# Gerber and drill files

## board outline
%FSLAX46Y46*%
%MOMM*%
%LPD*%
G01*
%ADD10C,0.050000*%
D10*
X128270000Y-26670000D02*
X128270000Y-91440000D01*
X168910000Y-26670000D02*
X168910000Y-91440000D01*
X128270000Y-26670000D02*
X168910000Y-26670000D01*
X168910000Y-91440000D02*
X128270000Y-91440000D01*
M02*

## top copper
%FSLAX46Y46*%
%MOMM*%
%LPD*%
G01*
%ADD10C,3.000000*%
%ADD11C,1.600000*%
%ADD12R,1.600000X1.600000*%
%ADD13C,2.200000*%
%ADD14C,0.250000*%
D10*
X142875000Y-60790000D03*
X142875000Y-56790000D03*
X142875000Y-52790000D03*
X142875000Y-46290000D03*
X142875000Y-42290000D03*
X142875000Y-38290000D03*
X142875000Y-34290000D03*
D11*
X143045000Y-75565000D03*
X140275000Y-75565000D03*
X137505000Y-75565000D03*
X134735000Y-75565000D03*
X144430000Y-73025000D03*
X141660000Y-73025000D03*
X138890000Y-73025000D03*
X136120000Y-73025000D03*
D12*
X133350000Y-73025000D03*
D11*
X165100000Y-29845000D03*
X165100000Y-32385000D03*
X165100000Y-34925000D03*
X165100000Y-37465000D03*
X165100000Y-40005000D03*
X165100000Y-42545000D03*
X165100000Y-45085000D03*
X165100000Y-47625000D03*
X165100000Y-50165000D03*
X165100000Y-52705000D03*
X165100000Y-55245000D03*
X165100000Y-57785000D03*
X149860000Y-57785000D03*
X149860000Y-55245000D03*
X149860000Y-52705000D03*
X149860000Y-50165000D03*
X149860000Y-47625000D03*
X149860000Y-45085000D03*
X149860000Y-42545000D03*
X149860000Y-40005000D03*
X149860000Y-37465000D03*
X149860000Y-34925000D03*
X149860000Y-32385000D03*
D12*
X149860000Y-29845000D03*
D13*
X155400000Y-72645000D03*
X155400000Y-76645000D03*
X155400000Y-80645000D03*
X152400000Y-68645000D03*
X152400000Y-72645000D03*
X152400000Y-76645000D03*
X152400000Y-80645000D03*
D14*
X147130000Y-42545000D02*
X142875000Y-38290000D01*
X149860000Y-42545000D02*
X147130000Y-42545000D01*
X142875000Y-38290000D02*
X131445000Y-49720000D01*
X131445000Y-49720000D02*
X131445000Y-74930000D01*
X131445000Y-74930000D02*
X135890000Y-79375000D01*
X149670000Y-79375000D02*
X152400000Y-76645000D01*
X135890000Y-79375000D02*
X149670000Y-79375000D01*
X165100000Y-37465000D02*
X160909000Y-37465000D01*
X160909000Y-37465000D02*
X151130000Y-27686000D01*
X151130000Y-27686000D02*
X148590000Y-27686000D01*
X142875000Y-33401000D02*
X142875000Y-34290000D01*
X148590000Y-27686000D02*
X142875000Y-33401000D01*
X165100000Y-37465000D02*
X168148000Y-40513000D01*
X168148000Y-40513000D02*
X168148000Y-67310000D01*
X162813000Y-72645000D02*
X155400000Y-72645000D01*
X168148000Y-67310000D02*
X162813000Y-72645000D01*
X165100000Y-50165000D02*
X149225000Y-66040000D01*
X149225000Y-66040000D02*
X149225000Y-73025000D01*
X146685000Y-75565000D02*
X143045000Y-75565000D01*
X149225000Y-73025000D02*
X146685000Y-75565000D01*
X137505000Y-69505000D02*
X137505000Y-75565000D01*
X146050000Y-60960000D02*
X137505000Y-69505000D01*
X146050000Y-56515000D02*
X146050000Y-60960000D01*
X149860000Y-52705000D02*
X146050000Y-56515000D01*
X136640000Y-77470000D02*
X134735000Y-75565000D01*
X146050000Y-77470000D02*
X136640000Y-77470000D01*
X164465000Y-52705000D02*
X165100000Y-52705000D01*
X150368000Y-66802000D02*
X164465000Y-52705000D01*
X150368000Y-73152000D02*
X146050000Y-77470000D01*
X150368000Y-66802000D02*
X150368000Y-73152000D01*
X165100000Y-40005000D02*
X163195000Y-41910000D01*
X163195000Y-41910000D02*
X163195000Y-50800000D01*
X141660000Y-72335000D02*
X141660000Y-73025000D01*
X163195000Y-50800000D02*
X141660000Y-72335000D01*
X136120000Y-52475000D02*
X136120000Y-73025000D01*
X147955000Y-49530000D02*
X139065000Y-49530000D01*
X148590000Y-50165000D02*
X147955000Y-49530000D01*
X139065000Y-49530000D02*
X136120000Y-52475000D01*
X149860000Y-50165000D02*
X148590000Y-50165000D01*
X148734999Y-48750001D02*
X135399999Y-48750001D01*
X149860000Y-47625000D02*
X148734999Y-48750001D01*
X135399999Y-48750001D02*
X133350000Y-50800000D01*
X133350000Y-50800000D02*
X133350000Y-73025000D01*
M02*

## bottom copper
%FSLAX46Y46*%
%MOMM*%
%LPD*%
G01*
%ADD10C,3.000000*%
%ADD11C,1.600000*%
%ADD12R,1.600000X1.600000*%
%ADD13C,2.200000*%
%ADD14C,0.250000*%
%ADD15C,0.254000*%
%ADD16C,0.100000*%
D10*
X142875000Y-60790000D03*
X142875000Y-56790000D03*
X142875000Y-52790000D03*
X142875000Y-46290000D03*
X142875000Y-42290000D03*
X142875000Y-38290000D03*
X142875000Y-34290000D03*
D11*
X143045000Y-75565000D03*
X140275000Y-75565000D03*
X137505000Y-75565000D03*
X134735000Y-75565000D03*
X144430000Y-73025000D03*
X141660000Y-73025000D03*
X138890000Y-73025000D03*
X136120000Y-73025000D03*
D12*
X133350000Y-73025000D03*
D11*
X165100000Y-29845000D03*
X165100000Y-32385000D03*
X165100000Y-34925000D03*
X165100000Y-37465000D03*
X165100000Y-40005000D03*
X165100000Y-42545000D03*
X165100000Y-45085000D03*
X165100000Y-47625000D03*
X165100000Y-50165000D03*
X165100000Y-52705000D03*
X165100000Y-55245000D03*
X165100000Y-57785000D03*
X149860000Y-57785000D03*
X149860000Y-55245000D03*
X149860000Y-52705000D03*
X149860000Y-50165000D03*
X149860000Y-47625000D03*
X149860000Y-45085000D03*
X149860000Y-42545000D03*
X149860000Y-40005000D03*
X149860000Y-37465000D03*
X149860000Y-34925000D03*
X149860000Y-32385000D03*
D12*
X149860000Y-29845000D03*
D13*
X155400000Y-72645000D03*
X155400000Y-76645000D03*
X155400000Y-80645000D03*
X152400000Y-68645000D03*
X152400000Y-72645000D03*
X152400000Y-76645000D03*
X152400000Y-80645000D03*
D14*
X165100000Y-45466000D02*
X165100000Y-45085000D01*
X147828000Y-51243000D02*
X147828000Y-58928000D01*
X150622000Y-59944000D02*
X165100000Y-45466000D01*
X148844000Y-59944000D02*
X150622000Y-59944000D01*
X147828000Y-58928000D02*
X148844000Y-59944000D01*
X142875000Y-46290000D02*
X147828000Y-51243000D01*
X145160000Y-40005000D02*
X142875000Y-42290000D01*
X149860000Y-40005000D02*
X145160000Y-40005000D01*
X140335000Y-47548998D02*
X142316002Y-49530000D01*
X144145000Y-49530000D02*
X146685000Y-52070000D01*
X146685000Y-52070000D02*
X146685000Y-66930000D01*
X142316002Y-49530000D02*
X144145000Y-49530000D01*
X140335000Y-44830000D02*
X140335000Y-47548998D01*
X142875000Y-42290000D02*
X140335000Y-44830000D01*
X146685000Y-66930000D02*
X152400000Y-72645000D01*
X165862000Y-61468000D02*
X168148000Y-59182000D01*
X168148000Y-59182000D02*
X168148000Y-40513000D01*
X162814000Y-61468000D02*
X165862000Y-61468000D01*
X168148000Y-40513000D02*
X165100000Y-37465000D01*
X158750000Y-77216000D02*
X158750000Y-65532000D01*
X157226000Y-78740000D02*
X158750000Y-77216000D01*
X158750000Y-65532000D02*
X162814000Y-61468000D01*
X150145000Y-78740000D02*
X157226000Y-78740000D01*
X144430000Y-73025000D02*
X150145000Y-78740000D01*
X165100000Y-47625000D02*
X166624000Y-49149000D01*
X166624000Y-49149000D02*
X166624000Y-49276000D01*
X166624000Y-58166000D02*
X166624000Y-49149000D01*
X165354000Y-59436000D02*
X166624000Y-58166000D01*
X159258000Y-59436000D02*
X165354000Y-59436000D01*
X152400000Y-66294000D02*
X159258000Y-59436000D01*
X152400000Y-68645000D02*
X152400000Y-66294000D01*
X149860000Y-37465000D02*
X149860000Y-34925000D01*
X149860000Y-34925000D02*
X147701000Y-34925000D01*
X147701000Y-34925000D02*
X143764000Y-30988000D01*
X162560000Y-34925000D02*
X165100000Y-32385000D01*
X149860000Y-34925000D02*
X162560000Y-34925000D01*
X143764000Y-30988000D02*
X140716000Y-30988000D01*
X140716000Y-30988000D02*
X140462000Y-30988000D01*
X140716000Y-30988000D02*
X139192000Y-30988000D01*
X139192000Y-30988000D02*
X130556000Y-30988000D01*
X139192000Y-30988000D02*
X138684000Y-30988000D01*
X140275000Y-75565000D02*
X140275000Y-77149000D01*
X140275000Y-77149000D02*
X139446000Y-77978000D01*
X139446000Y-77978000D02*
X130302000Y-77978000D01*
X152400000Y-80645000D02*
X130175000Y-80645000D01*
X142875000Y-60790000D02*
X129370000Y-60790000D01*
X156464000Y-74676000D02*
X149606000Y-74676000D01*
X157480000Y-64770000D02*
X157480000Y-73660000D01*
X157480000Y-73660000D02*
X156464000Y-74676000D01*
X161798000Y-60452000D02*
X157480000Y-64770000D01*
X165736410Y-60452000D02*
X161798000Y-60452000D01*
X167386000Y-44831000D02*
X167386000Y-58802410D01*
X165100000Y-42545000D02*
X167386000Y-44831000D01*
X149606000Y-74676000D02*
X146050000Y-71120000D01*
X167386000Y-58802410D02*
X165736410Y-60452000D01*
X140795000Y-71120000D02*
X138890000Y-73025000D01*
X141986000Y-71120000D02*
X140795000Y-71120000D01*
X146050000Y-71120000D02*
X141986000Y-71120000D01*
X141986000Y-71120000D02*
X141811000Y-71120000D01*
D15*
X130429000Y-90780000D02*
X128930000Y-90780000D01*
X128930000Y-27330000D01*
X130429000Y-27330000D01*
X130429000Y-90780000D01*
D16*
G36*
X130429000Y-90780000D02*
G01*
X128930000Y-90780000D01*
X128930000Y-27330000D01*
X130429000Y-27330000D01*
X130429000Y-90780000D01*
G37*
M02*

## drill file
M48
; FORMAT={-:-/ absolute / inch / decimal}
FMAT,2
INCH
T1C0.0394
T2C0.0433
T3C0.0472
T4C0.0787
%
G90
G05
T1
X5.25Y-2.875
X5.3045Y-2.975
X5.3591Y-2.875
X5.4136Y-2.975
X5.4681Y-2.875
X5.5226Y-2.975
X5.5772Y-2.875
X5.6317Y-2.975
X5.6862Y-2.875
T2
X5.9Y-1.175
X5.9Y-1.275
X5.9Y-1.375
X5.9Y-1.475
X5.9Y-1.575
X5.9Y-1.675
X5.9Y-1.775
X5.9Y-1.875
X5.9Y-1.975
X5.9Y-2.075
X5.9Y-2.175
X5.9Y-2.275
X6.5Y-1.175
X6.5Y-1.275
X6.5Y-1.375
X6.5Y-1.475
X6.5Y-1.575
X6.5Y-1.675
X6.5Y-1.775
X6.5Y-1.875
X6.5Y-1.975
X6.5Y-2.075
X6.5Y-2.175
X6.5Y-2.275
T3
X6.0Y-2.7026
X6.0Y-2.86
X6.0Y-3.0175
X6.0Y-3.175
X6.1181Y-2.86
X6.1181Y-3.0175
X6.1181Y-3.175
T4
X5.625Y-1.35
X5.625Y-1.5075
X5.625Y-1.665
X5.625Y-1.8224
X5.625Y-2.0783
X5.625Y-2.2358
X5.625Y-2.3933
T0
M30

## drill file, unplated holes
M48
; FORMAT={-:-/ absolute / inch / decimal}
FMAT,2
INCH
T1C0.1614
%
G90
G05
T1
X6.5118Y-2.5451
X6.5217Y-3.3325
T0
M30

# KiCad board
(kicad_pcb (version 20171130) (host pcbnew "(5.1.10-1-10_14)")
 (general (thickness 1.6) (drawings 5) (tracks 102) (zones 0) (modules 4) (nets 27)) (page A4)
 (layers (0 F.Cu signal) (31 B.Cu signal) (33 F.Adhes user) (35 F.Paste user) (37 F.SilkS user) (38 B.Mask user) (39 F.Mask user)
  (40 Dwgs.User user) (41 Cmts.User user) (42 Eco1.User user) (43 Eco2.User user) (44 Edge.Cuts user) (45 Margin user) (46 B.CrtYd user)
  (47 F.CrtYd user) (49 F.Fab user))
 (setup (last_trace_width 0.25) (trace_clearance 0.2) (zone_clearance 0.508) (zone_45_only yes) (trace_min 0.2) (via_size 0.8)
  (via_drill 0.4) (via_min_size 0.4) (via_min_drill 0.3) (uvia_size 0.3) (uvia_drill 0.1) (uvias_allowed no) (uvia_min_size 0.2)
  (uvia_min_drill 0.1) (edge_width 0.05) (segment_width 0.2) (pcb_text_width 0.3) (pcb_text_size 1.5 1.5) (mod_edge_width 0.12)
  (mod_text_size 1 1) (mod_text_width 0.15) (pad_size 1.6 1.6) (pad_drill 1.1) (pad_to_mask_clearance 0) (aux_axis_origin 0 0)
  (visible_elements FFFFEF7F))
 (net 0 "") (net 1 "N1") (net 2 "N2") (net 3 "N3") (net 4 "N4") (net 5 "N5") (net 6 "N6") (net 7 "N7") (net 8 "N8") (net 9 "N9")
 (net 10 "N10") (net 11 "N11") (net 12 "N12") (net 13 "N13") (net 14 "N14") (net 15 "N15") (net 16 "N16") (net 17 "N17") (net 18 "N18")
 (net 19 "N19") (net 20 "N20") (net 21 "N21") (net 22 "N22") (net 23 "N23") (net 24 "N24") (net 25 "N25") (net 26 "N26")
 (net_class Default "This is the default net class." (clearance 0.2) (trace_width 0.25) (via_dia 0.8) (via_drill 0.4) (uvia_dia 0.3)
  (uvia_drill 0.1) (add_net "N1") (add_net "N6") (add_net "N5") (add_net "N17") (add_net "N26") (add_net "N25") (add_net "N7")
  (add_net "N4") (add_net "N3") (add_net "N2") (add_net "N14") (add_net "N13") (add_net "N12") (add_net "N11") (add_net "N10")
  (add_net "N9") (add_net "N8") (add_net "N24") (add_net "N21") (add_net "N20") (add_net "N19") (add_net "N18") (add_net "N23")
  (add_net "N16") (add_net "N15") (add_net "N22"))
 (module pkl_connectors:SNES (layer F.Cu) (at 142.875 34.29 270)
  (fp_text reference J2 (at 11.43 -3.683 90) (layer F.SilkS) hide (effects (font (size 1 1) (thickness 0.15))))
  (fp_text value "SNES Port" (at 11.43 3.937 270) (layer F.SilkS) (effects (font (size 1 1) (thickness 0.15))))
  (pad 7 thru_hole circle (at 26.5 0 270) (size 3 3) (drill 2) (layers *.Cu *.Mask) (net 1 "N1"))
  (pad 6 thru_hole circle (at 22.5 0 270) (size 3 3) (drill 2) (layers *.Cu *.Mask) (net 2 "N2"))
  (pad 5 thru_hole circle (at 18.5 0 270) (size 3 3) (drill 2) (layers *.Cu *.Mask) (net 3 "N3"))
  (pad 4 thru_hole circle (at 12 0 270) (size 3 3) (drill 2) (layers *.Cu *.Mask) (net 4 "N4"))
  (pad 3 thru_hole circle (at 8 0 270) (size 3 3) (drill 2) (layers *.Cu *.Mask) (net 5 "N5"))
  (pad 2 thru_hole circle (at 4 0 270) (size 3 3) (drill 2) (layers *.Cu *.Mask) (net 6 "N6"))
  (pad 1 thru_hole circle (at 0 0 270) (size 3 3) (drill 2) (layers *.Cu *.Mask) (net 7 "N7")))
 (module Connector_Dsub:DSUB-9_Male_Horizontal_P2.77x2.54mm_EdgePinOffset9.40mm (layer F.Cu) (at 133.35 73.025)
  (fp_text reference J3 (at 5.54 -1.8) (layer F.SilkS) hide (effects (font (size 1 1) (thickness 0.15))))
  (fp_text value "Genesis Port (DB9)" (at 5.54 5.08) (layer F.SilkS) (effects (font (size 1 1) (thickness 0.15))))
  (pad 9 thru_hole circle (at 9.695 2.54) (size 1.6 1.6) (drill 1) (layers *.Cu *.Mask) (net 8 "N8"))
  (pad 8 thru_hole circle (at 6.925 2.54) (size 1.6 1.6) (drill 1) (layers *.Cu *.Mask) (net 1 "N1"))
  (pad 7 thru_hole circle (at 4.155 2.54) (size 1.6 1.6) (drill 1) (layers *.Cu *.Mask) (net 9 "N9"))
  (pad 6 thru_hole circle (at 1.385 2.54) (size 1.6 1.6) (drill 1) (layers *.Cu *.Mask) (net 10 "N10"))
  (pad 5 thru_hole circle (at 11.08 0) (size 1.6 1.6) (drill 1) (layers *.Cu *.Mask) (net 7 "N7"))
  (pad 4 thru_hole circle (at 8.31 0) (size 1.6 1.6) (drill 1) (layers *.Cu *.Mask) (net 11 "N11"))
  (pad 3 thru_hole circle (at 5.54 0) (size 1.6 1.6) (drill 1) (layers *.Cu *.Mask) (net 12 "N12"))
  (pad 2 thru_hole circle (at 2.77 0) (size 1.6 1.6) (drill 1) (layers *.Cu *.Mask) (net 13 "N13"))
  (pad 1 thru_hole rect (at 0 0) (size 1.6 1.6) (drill 1) (layers *.Cu *.Mask) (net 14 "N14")))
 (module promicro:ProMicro (layer F.Cu) (at 157.48 43.815 270)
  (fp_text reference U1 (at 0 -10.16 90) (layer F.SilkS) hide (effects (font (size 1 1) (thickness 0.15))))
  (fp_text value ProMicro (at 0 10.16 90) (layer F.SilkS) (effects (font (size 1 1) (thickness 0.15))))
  (pad 24 thru_hole circle (at -13.97 -7.62 270) (size 1.6 1.6) (drill 1.1) (layers *.Cu *.Mask F.SilkS) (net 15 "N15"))
  (pad 23 thru_hole circle (at -11.43 -7.62 270) (size 1.6 1.6) (drill 1.1) (layers *.Cu *.Mask F.SilkS) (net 1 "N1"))
  (pad 22 thru_hole circle (at -8.89 -7.62 270) (size 1.6 1.6) (drill 1.1) (layers *.Cu *.Mask F.SilkS) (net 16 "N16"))
  (pad 21 thru_hole circle (at -6.35 -7.62 270) (size 1.6 1.6) (drill 1.1) (layers *.Cu *.Mask F.SilkS) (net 7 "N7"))
  (pad 20 thru_hole circle (at -3.81 -7.62 270) (size 1.6 1.6) (drill 1.1) (layers *.Cu *.Mask F.SilkS) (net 11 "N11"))
  (pad 19 thru_hole circle (at -1.27 -7.62 270) (size 1.6 1.6) (drill 1.1) (layers *.Cu *.Mask F.SilkS) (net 12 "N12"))
  (pad 18 thru_hole circle (at 1.27 -7.62 270) (size 1.6 1.6) (drill 1.1) (layers *.Cu *.Mask F.SilkS) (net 4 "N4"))
  (pad 17 thru_hole circle (at 3.81 -7.62 270) (size 1.6 1.6) (drill 1.1) (layers *.Cu *.Mask F.SilkS) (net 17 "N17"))
  (pad 16 thru_hole circle (at 6.35 -7.62 270) (size 1.6 1.6) (drill 1.1) (layers *.Cu *.Mask F.SilkS) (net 8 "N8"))
  (pad 15 thru_hole circle (at 8.89 -7.62 270) (size 1.6 1.6) (drill 1.1) (layers *.Cu *.Mask F.SilkS) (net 10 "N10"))
  (pad 14 thru_hole circle (at 11.43 -7.62 270) (size 1.6 1.6) (drill 1.1) (layers *.Cu *.Mask F.SilkS) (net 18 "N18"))
  (pad 13 thru_hole circle (at 13.97 -7.62 270) (size 1.6 1.6) (drill 1.1) (layers *.Cu *.Mask F.SilkS) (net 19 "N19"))
  (pad 12 thru_hole circle (at 13.97 7.62 270) (size 1.6 1.6) (drill 1.1) (layers *.Cu *.Mask F.SilkS) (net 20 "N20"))
  (pad 11 thru_hole circle (at 11.43 7.62 270) (size 1.6 1.6) (drill 1.1) (layers *.Cu *.Mask F.SilkS) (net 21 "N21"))
  (pad 10 thru_hole circle (at 8.89 7.62 270) (size 1.6 1.6) (drill 1.1) (layers *.Cu *.Mask F.SilkS) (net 9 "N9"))
  (pad 9 thru_hole circle (at 6.35 7.62 270) (size 1.6 1.6) (drill 1.1) (layers *.Cu *.Mask F.SilkS) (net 13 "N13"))
  (pad 8 thru_hole circle (at 3.81 7.62 270) (size 1.6 1.6) (drill 1.1) (layers *.Cu *.Mask F.SilkS) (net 14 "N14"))
  (pad 7 thru_hole circle (at 1.27 7.62 270) (size 1.6 1.6) (drill 1.1) (layers *.Cu *.Mask F.SilkS) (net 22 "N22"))
  (pad 6 thru_hole circle (at -1.27 7.62 270) (size 1.6 1.6) (drill 1.1) (layers *.Cu *.Mask F.SilkS) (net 6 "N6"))
  (pad 5 thru_hole circle (at -3.81 7.62 270) (size 1.6 1.6) (drill 1.1) (layers *.Cu *.Mask F.SilkS) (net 5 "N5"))
  (pad 4 thru_hole circle (at -6.35 7.62 270) (size 1.6 1.6) (drill 1.1) (layers *.Cu *.Mask F.SilkS) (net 1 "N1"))
  (pad 3 thru_hole circle (at -8.89 7.62 270) (size 1.6 1.6) (drill 1.1) (layers *.Cu *.Mask F.SilkS) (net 1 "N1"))
  (pad 2 thru_hole circle (at -11.43 7.62 270) (size 1.6 1.6) (drill 1.1) (layers *.Cu *.Mask F.SilkS) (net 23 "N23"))
  (pad 1 thru_hole rect (at -13.97 7.62 270) (size 1.6 1.6) (drill 1.1) (layers *.Cu *.Mask F.SilkS) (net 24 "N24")))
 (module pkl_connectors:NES (layer F.Cu) (at 152.4 80.645 90)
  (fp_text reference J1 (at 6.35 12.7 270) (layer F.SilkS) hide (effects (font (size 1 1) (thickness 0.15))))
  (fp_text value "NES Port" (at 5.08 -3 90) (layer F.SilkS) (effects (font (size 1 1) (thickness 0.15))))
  (pad "" np_thru_hole circle (at -4 13.25 90) (size 4.1 4.1) (drill 4.1) (layers *.Cu *.Mask))
  (pad "" np_thru_hole circle (at 16 13 90) (size 4.1 4.1) (drill 4.1) (layers *.Cu *.Mask))
  (pad 7 thru_hole circle (at 8 3 90) (size 2.2 2.2) (drill 1.2) (layers *.Cu *.Mask) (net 7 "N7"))
  (pad 6 thru_hole circle (at 4 3 90) (size 2.2 2.2) (drill 1.2) (layers *.Cu *.Mask) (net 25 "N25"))
  (pad 5 thru_hole circle (at 0 3 90) (size 2.2 2.2) (drill 1.2) (layers *.Cu *.Mask) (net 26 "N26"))
  (pad 4 thru_hole circle (at 12 0 90) (size 2.2 2.2) (drill 1.2) (layers *.Cu *.Mask) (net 17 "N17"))
  (pad 3 thru_hole circle (at 8 0 90) (size 2.2 2.2) (drill 1.2) (layers *.Cu *.Mask) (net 5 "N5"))
  (pad 2 thru_hole circle (at 4 0 90) (size 2.2 2.2) (drill 1.2) (layers *.Cu *.Mask) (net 6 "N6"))
  (pad 1 thru_hole circle (at 0 0 90) (size 2.2 2.2) (drill 1.2) (layers *.Cu *.Mask) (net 1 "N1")))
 (gr_line (start 128.27 26.67) (end 128.27 91.44) (layer Edge.Cuts) (width 0.05))
 (gr_line (start 168.91 26.67) (end 168.91 91.44) (layer Edge.Cuts) (width 0.05))
 (gr_line (start 128.27 26.67) (end 168.91 26.67) (layer Edge.Cuts) (width 0.05))
 (gr_line (start 168.91 91.44) (end 128.27 91.44) (layer Edge.Cuts) (width 0.05))
 (segment (start 165.1 45.466) (end 165.1 45.085) (width 0.25) (layer B.Cu) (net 4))
 (segment (start 147.828 51.243) (end 147.828 58.928) (width 0.25) (layer B.Cu) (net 4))
 (segment (start 150.622 59.944) (end 165.1 45.466) (width 0.25) (layer B.Cu) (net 4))
 (segment (start 148.844 59.944) (end 150.622 59.944) (width 0.25) (layer B.Cu) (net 4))
 (segment (start 147.828 58.928) (end 148.844 59.944) (width 0.25) (layer B.Cu) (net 4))
 (segment (start 142.875 46.29) (end 147.828 51.243) (width 0.25) (layer B.Cu) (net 4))
 (segment (start 145.16 40.005) (end 142.875 42.29) (width 0.25) (layer B.Cu) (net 5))
 (segment (start 149.86 40.005) (end 145.16 40.005) (width 0.25) (layer B.Cu) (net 5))
 (segment (start 140.335 47.548998) (end 142.316002 49.53) (width 0.25) (layer B.Cu) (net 5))
 (segment (start 144.145 49.53) (end 146.685 52.07) (width 0.25) (layer B.Cu) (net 5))
 (segment (start 146.685 52.07) (end 146.685 66.93) (width 0.25) (layer B.Cu) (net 5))
 (segment (start 142.316002 49.53) (end 144.145 49.53) (width 0.25) (layer B.Cu) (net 5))
 (segment (start 140.335 44.83) (end 140.335 47.548998) (width 0.25) (layer B.Cu) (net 5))
 (segment (start 142.875 42.29) (end 140.335 44.83) (width 0.25) (layer B.Cu) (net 5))
 (segment (start 146.685 66.93) (end 152.4 72.645) (width 0.25) (layer B.Cu) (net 5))
 (segment (start 147.13 42.545) (end 142.875 38.29) (width 0.25) (layer F.Cu) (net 6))
 (segment (start 149.86 42.545) (end 147.13 42.545) (width 0.25) (layer F.Cu) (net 6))
 (segment (start 142.875 38.29) (end 131.445 49.72) (width 0.25) (layer F.Cu) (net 6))
 (segment (start 131.445 49.72) (end 131.445 74.93) (width 0.25) (layer F.Cu) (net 6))
 (segment (start 131.445 74.93) (end 135.89 79.375) (width 0.25) (layer F.Cu) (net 6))
 (segment (start 149.67 79.375) (end 152.4 76.645) (width 0.25) (layer F.Cu) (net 6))
 (segment (start 135.89 79.375) (end 149.67 79.375) (width 0.25) (layer F.Cu) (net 6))
 (segment (start 165.1 37.465) (end 160.909 37.465) (width 0.25) (layer F.Cu) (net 7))
 (segment (start 160.909 37.465) (end 151.13 27.686) (width 0.25) (layer F.Cu) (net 7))
 (segment (start 151.13 27.686) (end 148.59 27.686) (width 0.25) (layer F.Cu) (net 7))
 (segment (start 142.875 33.401) (end 142.875 34.29) (width 0.25) (layer F.Cu) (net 7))
 (segment (start 148.59 27.686) (end 142.875 33.401) (width 0.25) (layer F.Cu) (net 7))
 (segment (start 165.1 37.465) (end 168.148 40.513) (width 0.25) (layer F.Cu) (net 7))
 (segment (start 168.148 40.513) (end 168.148 67.31) (width 0.25) (layer F.Cu) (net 7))
 (segment (start 162.813 72.645) (end 155.4 72.645) (width 0.25) (layer F.Cu) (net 7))
 (segment (start 168.148 67.31) (end 162.813 72.645) (width 0.25) (layer F.Cu) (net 7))
 (segment (start 165.862 61.468) (end 168.148 59.182) (width 0.25) (layer B.Cu) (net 7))
 (segment (start 168.148 59.182) (end 168.148 40.513) (width 0.25) (layer B.Cu) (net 7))
 (segment (start 162.814 61.468) (end 165.862 61.468) (width 0.25) (layer B.Cu) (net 7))
 (segment (start 168.148 40.513) (end 165.1 37.465) (width 0.25) (layer B.Cu) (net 7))
 (segment (start 158.75 77.216) (end 158.75 65.532) (width 0.25) (layer B.Cu) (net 7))
 (segment (start 157.226 78.74) (end 158.75 77.216) (width 0.25) (layer B.Cu) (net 7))
 (segment (start 158.75 65.532) (end 162.814 61.468) (width 0.25) (layer B.Cu) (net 7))
 (segment (start 150.145 78.74) (end 157.226 78.74) (width 0.25) (layer B.Cu) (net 7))
 (segment (start 144.43 73.025) (end 150.145 78.74) (width 0.25) (layer B.Cu) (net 7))
 (segment (start 165.1 47.625) (end 166.624 49.149) (width 0.25) (layer B.Cu) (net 17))
 (segment (start 166.624 49.149) (end 166.624 49.276) (width 0.25) (layer B.Cu) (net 17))
 (segment (start 166.624 58.166) (end 166.624 49.149) (width 0.25) (layer B.Cu) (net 17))
 (segment (start 165.354 59.436) (end 166.624 58.166) (width 0.25) (layer B.Cu) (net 17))
 (segment (start 159.258 59.436) (end 165.354 59.436) (width 0.25) (layer B.Cu) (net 17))
 (segment (start 152.4 66.294) (end 159.258 59.436) (width 0.25) (layer B.Cu) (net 17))
 (segment (start 152.4 68.645) (end 152.4 66.294) (width 0.25) (layer B.Cu) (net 17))
 (segment (start 149.86 37.465) (end 149.86 34.925) (width 0.25) (layer B.Cu) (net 1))
 (segment (start 149.86 34.925) (end 147.701 34.925) (width 0.25) (layer B.Cu) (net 1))
 (segment (start 147.701 34.925) (end 143.764 30.988) (width 0.25) (layer B.Cu) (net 1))
 (segment (start 162.56 34.925) (end 165.1 32.385) (width 0.25) (layer B.Cu) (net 1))
 (segment (start 149.86 34.925) (end 162.56 34.925) (width 0.25) (layer B.Cu) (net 1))
 (segment (start 143.764 30.988) (end 140.716 30.988) (width 0.25) (layer B.Cu) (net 1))
 (segment (start 140.716 30.988) (end 140.462 30.988) (width 0.25) (layer B.Cu) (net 1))
 (segment (start 140.716 30.988) (end 139.192 30.988) (width 0.25) (layer B.Cu) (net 1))
 (segment (start 139.192 30.988) (end 130.556 30.988) (width 0.25) (layer B.Cu) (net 1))
 (segment (start 139.192 30.988) (end 138.684 30.988) (width 0.25) (layer B.Cu) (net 1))
 (segment (start 140.275 75.565) (end 140.275 77.149) (width 0.25) (layer B.Cu) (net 1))
 (segment (start 140.275 77.149) (end 139.446 77.978) (width 0.25) (layer B.Cu) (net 1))
 (segment (start 139.446 77.978) (end 130.302 77.978) (width 0.25) (layer B.Cu) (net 1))
 (segment (start 152.4 80.645) (end 130.175 80.645) (width 0.25) (layer B.Cu) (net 1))
 (segment (start 142.875 60.79) (end 129.37 60.79) (width 0.25) (layer B.Cu) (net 1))
 (segment (start 165.1 50.165) (end 149.225 66.04) (width 0.25) (layer F.Cu) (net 8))
 (segment (start 149.225 66.04) (end 149.225 73.025) (width 0.25) (layer F.Cu) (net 8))
 (segment (start 146.685 75.565) (end 143.045 75.565) (width 0.25) (layer F.Cu) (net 8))
 (segment (start 149.225 73.025) (end 146.685 75.565) (width 0.25) (layer F.Cu) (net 8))
 (segment (start 137.505 69.505) (end 137.505 75.565) (width 0.25) (layer F.Cu) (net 9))
 (segment (start 146.05 60.96) (end 137.505 69.505) (width 0.25) (layer F.Cu) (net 9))
 (segment (start 146.05 56.515) (end 146.05 60.96) (width 0.25) (layer F.Cu) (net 9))
 (segment (start 149.86 52.705) (end 146.05 56.515) (width 0.25) (layer F.Cu) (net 9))
 (segment (start 136.64 77.47) (end 134.735 75.565) (width 0.25) (layer F.Cu) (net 10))
 (segment (start 146.05 77.47) (end 136.64 77.47) (width 0.25) (layer F.Cu) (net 10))
 (segment (start 164.465 52.705) (end 165.1 52.705) (width 0.25) (layer F.Cu) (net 10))
 (segment (start 150.368 66.802) (end 164.465 52.705) (width 0.25) (layer F.Cu) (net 10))
 (segment (start 150.368 73.152) (end 146.05 77.47) (width 0.25) (layer F.Cu) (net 10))
 (segment (start 150.368 66.802) (end 150.368 73.152) (width 0.25) (layer F.Cu) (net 10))
 (segment (start 165.1 40.005) (end 163.195 41.91) (width 0.25) (layer F.Cu) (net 11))
 (segment (start 163.195 41.91) (end 163.195 50.8) (width 0.25) (layer F.Cu) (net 11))
 (segment (start 141.66 72.335) (end 141.66 73.025) (width 0.25) (layer F.Cu) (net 11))
 (segment (start 163.195 50.8) (end 141.66 72.335) (width 0.25) (layer F.Cu) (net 11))
 (segment (start 156.464 74.676) (end 149.606 74.676) (width 0.25) (layer B.Cu) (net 12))
 (segment (start 157.48 64.77) (end 157.48 73.66) (width 0.25) (layer B.Cu) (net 12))
 (segment (start 157.48 73.66) (end 156.464 74.676) (width 0.25) (layer B.Cu) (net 12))
 (segment (start 161.798 60.452) (end 157.48 64.77) (width 0.25) (layer B.Cu) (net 12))
 (segment (start 165.73641 60.452) (end 161.798 60.452) (width 0.25) (layer B.Cu) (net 12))
 (segment (start 167.386 44.831) (end 167.386 58.80241) (width 0.25) (layer B.Cu) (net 12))
 (segment (start 165.1 42.545) (end 167.386 44.831) (width 0.25) (layer B.Cu) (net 12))
 (segment (start 149.606 74.676) (end 146.05 71.12) (width 0.25) (layer B.Cu) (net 12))
 (segment (start 167.386 58.80241) (end 165.73641 60.452) (width 0.25) (layer B.Cu) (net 12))
 (segment (start 140.795 71.12) (end 138.89 73.025) (width 0.25) (layer B.Cu) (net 12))
 (segment (start 141.986 71.12) (end 140.795 71.12) (width 0.25) (layer B.Cu) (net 12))
 (segment (start 146.05 71.12) (end 141.986 71.12) (width 0.25) (layer B.Cu) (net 12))
 (segment (start 141.986 71.12) (end 141.811 71.12) (width 0.25) (layer B.Cu) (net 12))
 (segment (start 136.12 52.475) (end 136.12 73.025) (width 0.25) (layer F.Cu) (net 13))
 (segment (start 147.955 49.53) (end 139.065 49.53) (width 0.25) (layer F.Cu) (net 13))
 (segment (start 148.59 50.165) (end 147.955 49.53) (width 0.25) (layer F.Cu) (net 13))
 (segment (start 139.065 49.53) (end 136.12 52.475) (width 0.25) (layer F.Cu) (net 13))
 (segment (start 149.86 50.165) (end 148.59 50.165) (width 0.25) (layer F.Cu) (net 13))
 (segment (start 148.734999 48.750001) (end 135.399999 48.750001) (width 0.25) (layer F.Cu) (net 14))
 (segment (start 149.86 47.625) (end 148.734999 48.750001) (width 0.25) (layer F.Cu) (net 14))
 (segment (start 135.399999 48.750001) (end 133.35 50.8) (width 0.25) (layer F.Cu) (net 14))
 (segment (start 133.35 50.8) (end 133.35 73.025) (width 0.25) (layer F.Cu) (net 14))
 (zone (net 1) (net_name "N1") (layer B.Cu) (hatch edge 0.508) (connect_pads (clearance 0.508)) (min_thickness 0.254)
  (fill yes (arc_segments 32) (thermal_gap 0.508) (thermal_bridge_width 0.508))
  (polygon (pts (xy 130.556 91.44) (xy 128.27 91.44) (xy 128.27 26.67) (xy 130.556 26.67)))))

